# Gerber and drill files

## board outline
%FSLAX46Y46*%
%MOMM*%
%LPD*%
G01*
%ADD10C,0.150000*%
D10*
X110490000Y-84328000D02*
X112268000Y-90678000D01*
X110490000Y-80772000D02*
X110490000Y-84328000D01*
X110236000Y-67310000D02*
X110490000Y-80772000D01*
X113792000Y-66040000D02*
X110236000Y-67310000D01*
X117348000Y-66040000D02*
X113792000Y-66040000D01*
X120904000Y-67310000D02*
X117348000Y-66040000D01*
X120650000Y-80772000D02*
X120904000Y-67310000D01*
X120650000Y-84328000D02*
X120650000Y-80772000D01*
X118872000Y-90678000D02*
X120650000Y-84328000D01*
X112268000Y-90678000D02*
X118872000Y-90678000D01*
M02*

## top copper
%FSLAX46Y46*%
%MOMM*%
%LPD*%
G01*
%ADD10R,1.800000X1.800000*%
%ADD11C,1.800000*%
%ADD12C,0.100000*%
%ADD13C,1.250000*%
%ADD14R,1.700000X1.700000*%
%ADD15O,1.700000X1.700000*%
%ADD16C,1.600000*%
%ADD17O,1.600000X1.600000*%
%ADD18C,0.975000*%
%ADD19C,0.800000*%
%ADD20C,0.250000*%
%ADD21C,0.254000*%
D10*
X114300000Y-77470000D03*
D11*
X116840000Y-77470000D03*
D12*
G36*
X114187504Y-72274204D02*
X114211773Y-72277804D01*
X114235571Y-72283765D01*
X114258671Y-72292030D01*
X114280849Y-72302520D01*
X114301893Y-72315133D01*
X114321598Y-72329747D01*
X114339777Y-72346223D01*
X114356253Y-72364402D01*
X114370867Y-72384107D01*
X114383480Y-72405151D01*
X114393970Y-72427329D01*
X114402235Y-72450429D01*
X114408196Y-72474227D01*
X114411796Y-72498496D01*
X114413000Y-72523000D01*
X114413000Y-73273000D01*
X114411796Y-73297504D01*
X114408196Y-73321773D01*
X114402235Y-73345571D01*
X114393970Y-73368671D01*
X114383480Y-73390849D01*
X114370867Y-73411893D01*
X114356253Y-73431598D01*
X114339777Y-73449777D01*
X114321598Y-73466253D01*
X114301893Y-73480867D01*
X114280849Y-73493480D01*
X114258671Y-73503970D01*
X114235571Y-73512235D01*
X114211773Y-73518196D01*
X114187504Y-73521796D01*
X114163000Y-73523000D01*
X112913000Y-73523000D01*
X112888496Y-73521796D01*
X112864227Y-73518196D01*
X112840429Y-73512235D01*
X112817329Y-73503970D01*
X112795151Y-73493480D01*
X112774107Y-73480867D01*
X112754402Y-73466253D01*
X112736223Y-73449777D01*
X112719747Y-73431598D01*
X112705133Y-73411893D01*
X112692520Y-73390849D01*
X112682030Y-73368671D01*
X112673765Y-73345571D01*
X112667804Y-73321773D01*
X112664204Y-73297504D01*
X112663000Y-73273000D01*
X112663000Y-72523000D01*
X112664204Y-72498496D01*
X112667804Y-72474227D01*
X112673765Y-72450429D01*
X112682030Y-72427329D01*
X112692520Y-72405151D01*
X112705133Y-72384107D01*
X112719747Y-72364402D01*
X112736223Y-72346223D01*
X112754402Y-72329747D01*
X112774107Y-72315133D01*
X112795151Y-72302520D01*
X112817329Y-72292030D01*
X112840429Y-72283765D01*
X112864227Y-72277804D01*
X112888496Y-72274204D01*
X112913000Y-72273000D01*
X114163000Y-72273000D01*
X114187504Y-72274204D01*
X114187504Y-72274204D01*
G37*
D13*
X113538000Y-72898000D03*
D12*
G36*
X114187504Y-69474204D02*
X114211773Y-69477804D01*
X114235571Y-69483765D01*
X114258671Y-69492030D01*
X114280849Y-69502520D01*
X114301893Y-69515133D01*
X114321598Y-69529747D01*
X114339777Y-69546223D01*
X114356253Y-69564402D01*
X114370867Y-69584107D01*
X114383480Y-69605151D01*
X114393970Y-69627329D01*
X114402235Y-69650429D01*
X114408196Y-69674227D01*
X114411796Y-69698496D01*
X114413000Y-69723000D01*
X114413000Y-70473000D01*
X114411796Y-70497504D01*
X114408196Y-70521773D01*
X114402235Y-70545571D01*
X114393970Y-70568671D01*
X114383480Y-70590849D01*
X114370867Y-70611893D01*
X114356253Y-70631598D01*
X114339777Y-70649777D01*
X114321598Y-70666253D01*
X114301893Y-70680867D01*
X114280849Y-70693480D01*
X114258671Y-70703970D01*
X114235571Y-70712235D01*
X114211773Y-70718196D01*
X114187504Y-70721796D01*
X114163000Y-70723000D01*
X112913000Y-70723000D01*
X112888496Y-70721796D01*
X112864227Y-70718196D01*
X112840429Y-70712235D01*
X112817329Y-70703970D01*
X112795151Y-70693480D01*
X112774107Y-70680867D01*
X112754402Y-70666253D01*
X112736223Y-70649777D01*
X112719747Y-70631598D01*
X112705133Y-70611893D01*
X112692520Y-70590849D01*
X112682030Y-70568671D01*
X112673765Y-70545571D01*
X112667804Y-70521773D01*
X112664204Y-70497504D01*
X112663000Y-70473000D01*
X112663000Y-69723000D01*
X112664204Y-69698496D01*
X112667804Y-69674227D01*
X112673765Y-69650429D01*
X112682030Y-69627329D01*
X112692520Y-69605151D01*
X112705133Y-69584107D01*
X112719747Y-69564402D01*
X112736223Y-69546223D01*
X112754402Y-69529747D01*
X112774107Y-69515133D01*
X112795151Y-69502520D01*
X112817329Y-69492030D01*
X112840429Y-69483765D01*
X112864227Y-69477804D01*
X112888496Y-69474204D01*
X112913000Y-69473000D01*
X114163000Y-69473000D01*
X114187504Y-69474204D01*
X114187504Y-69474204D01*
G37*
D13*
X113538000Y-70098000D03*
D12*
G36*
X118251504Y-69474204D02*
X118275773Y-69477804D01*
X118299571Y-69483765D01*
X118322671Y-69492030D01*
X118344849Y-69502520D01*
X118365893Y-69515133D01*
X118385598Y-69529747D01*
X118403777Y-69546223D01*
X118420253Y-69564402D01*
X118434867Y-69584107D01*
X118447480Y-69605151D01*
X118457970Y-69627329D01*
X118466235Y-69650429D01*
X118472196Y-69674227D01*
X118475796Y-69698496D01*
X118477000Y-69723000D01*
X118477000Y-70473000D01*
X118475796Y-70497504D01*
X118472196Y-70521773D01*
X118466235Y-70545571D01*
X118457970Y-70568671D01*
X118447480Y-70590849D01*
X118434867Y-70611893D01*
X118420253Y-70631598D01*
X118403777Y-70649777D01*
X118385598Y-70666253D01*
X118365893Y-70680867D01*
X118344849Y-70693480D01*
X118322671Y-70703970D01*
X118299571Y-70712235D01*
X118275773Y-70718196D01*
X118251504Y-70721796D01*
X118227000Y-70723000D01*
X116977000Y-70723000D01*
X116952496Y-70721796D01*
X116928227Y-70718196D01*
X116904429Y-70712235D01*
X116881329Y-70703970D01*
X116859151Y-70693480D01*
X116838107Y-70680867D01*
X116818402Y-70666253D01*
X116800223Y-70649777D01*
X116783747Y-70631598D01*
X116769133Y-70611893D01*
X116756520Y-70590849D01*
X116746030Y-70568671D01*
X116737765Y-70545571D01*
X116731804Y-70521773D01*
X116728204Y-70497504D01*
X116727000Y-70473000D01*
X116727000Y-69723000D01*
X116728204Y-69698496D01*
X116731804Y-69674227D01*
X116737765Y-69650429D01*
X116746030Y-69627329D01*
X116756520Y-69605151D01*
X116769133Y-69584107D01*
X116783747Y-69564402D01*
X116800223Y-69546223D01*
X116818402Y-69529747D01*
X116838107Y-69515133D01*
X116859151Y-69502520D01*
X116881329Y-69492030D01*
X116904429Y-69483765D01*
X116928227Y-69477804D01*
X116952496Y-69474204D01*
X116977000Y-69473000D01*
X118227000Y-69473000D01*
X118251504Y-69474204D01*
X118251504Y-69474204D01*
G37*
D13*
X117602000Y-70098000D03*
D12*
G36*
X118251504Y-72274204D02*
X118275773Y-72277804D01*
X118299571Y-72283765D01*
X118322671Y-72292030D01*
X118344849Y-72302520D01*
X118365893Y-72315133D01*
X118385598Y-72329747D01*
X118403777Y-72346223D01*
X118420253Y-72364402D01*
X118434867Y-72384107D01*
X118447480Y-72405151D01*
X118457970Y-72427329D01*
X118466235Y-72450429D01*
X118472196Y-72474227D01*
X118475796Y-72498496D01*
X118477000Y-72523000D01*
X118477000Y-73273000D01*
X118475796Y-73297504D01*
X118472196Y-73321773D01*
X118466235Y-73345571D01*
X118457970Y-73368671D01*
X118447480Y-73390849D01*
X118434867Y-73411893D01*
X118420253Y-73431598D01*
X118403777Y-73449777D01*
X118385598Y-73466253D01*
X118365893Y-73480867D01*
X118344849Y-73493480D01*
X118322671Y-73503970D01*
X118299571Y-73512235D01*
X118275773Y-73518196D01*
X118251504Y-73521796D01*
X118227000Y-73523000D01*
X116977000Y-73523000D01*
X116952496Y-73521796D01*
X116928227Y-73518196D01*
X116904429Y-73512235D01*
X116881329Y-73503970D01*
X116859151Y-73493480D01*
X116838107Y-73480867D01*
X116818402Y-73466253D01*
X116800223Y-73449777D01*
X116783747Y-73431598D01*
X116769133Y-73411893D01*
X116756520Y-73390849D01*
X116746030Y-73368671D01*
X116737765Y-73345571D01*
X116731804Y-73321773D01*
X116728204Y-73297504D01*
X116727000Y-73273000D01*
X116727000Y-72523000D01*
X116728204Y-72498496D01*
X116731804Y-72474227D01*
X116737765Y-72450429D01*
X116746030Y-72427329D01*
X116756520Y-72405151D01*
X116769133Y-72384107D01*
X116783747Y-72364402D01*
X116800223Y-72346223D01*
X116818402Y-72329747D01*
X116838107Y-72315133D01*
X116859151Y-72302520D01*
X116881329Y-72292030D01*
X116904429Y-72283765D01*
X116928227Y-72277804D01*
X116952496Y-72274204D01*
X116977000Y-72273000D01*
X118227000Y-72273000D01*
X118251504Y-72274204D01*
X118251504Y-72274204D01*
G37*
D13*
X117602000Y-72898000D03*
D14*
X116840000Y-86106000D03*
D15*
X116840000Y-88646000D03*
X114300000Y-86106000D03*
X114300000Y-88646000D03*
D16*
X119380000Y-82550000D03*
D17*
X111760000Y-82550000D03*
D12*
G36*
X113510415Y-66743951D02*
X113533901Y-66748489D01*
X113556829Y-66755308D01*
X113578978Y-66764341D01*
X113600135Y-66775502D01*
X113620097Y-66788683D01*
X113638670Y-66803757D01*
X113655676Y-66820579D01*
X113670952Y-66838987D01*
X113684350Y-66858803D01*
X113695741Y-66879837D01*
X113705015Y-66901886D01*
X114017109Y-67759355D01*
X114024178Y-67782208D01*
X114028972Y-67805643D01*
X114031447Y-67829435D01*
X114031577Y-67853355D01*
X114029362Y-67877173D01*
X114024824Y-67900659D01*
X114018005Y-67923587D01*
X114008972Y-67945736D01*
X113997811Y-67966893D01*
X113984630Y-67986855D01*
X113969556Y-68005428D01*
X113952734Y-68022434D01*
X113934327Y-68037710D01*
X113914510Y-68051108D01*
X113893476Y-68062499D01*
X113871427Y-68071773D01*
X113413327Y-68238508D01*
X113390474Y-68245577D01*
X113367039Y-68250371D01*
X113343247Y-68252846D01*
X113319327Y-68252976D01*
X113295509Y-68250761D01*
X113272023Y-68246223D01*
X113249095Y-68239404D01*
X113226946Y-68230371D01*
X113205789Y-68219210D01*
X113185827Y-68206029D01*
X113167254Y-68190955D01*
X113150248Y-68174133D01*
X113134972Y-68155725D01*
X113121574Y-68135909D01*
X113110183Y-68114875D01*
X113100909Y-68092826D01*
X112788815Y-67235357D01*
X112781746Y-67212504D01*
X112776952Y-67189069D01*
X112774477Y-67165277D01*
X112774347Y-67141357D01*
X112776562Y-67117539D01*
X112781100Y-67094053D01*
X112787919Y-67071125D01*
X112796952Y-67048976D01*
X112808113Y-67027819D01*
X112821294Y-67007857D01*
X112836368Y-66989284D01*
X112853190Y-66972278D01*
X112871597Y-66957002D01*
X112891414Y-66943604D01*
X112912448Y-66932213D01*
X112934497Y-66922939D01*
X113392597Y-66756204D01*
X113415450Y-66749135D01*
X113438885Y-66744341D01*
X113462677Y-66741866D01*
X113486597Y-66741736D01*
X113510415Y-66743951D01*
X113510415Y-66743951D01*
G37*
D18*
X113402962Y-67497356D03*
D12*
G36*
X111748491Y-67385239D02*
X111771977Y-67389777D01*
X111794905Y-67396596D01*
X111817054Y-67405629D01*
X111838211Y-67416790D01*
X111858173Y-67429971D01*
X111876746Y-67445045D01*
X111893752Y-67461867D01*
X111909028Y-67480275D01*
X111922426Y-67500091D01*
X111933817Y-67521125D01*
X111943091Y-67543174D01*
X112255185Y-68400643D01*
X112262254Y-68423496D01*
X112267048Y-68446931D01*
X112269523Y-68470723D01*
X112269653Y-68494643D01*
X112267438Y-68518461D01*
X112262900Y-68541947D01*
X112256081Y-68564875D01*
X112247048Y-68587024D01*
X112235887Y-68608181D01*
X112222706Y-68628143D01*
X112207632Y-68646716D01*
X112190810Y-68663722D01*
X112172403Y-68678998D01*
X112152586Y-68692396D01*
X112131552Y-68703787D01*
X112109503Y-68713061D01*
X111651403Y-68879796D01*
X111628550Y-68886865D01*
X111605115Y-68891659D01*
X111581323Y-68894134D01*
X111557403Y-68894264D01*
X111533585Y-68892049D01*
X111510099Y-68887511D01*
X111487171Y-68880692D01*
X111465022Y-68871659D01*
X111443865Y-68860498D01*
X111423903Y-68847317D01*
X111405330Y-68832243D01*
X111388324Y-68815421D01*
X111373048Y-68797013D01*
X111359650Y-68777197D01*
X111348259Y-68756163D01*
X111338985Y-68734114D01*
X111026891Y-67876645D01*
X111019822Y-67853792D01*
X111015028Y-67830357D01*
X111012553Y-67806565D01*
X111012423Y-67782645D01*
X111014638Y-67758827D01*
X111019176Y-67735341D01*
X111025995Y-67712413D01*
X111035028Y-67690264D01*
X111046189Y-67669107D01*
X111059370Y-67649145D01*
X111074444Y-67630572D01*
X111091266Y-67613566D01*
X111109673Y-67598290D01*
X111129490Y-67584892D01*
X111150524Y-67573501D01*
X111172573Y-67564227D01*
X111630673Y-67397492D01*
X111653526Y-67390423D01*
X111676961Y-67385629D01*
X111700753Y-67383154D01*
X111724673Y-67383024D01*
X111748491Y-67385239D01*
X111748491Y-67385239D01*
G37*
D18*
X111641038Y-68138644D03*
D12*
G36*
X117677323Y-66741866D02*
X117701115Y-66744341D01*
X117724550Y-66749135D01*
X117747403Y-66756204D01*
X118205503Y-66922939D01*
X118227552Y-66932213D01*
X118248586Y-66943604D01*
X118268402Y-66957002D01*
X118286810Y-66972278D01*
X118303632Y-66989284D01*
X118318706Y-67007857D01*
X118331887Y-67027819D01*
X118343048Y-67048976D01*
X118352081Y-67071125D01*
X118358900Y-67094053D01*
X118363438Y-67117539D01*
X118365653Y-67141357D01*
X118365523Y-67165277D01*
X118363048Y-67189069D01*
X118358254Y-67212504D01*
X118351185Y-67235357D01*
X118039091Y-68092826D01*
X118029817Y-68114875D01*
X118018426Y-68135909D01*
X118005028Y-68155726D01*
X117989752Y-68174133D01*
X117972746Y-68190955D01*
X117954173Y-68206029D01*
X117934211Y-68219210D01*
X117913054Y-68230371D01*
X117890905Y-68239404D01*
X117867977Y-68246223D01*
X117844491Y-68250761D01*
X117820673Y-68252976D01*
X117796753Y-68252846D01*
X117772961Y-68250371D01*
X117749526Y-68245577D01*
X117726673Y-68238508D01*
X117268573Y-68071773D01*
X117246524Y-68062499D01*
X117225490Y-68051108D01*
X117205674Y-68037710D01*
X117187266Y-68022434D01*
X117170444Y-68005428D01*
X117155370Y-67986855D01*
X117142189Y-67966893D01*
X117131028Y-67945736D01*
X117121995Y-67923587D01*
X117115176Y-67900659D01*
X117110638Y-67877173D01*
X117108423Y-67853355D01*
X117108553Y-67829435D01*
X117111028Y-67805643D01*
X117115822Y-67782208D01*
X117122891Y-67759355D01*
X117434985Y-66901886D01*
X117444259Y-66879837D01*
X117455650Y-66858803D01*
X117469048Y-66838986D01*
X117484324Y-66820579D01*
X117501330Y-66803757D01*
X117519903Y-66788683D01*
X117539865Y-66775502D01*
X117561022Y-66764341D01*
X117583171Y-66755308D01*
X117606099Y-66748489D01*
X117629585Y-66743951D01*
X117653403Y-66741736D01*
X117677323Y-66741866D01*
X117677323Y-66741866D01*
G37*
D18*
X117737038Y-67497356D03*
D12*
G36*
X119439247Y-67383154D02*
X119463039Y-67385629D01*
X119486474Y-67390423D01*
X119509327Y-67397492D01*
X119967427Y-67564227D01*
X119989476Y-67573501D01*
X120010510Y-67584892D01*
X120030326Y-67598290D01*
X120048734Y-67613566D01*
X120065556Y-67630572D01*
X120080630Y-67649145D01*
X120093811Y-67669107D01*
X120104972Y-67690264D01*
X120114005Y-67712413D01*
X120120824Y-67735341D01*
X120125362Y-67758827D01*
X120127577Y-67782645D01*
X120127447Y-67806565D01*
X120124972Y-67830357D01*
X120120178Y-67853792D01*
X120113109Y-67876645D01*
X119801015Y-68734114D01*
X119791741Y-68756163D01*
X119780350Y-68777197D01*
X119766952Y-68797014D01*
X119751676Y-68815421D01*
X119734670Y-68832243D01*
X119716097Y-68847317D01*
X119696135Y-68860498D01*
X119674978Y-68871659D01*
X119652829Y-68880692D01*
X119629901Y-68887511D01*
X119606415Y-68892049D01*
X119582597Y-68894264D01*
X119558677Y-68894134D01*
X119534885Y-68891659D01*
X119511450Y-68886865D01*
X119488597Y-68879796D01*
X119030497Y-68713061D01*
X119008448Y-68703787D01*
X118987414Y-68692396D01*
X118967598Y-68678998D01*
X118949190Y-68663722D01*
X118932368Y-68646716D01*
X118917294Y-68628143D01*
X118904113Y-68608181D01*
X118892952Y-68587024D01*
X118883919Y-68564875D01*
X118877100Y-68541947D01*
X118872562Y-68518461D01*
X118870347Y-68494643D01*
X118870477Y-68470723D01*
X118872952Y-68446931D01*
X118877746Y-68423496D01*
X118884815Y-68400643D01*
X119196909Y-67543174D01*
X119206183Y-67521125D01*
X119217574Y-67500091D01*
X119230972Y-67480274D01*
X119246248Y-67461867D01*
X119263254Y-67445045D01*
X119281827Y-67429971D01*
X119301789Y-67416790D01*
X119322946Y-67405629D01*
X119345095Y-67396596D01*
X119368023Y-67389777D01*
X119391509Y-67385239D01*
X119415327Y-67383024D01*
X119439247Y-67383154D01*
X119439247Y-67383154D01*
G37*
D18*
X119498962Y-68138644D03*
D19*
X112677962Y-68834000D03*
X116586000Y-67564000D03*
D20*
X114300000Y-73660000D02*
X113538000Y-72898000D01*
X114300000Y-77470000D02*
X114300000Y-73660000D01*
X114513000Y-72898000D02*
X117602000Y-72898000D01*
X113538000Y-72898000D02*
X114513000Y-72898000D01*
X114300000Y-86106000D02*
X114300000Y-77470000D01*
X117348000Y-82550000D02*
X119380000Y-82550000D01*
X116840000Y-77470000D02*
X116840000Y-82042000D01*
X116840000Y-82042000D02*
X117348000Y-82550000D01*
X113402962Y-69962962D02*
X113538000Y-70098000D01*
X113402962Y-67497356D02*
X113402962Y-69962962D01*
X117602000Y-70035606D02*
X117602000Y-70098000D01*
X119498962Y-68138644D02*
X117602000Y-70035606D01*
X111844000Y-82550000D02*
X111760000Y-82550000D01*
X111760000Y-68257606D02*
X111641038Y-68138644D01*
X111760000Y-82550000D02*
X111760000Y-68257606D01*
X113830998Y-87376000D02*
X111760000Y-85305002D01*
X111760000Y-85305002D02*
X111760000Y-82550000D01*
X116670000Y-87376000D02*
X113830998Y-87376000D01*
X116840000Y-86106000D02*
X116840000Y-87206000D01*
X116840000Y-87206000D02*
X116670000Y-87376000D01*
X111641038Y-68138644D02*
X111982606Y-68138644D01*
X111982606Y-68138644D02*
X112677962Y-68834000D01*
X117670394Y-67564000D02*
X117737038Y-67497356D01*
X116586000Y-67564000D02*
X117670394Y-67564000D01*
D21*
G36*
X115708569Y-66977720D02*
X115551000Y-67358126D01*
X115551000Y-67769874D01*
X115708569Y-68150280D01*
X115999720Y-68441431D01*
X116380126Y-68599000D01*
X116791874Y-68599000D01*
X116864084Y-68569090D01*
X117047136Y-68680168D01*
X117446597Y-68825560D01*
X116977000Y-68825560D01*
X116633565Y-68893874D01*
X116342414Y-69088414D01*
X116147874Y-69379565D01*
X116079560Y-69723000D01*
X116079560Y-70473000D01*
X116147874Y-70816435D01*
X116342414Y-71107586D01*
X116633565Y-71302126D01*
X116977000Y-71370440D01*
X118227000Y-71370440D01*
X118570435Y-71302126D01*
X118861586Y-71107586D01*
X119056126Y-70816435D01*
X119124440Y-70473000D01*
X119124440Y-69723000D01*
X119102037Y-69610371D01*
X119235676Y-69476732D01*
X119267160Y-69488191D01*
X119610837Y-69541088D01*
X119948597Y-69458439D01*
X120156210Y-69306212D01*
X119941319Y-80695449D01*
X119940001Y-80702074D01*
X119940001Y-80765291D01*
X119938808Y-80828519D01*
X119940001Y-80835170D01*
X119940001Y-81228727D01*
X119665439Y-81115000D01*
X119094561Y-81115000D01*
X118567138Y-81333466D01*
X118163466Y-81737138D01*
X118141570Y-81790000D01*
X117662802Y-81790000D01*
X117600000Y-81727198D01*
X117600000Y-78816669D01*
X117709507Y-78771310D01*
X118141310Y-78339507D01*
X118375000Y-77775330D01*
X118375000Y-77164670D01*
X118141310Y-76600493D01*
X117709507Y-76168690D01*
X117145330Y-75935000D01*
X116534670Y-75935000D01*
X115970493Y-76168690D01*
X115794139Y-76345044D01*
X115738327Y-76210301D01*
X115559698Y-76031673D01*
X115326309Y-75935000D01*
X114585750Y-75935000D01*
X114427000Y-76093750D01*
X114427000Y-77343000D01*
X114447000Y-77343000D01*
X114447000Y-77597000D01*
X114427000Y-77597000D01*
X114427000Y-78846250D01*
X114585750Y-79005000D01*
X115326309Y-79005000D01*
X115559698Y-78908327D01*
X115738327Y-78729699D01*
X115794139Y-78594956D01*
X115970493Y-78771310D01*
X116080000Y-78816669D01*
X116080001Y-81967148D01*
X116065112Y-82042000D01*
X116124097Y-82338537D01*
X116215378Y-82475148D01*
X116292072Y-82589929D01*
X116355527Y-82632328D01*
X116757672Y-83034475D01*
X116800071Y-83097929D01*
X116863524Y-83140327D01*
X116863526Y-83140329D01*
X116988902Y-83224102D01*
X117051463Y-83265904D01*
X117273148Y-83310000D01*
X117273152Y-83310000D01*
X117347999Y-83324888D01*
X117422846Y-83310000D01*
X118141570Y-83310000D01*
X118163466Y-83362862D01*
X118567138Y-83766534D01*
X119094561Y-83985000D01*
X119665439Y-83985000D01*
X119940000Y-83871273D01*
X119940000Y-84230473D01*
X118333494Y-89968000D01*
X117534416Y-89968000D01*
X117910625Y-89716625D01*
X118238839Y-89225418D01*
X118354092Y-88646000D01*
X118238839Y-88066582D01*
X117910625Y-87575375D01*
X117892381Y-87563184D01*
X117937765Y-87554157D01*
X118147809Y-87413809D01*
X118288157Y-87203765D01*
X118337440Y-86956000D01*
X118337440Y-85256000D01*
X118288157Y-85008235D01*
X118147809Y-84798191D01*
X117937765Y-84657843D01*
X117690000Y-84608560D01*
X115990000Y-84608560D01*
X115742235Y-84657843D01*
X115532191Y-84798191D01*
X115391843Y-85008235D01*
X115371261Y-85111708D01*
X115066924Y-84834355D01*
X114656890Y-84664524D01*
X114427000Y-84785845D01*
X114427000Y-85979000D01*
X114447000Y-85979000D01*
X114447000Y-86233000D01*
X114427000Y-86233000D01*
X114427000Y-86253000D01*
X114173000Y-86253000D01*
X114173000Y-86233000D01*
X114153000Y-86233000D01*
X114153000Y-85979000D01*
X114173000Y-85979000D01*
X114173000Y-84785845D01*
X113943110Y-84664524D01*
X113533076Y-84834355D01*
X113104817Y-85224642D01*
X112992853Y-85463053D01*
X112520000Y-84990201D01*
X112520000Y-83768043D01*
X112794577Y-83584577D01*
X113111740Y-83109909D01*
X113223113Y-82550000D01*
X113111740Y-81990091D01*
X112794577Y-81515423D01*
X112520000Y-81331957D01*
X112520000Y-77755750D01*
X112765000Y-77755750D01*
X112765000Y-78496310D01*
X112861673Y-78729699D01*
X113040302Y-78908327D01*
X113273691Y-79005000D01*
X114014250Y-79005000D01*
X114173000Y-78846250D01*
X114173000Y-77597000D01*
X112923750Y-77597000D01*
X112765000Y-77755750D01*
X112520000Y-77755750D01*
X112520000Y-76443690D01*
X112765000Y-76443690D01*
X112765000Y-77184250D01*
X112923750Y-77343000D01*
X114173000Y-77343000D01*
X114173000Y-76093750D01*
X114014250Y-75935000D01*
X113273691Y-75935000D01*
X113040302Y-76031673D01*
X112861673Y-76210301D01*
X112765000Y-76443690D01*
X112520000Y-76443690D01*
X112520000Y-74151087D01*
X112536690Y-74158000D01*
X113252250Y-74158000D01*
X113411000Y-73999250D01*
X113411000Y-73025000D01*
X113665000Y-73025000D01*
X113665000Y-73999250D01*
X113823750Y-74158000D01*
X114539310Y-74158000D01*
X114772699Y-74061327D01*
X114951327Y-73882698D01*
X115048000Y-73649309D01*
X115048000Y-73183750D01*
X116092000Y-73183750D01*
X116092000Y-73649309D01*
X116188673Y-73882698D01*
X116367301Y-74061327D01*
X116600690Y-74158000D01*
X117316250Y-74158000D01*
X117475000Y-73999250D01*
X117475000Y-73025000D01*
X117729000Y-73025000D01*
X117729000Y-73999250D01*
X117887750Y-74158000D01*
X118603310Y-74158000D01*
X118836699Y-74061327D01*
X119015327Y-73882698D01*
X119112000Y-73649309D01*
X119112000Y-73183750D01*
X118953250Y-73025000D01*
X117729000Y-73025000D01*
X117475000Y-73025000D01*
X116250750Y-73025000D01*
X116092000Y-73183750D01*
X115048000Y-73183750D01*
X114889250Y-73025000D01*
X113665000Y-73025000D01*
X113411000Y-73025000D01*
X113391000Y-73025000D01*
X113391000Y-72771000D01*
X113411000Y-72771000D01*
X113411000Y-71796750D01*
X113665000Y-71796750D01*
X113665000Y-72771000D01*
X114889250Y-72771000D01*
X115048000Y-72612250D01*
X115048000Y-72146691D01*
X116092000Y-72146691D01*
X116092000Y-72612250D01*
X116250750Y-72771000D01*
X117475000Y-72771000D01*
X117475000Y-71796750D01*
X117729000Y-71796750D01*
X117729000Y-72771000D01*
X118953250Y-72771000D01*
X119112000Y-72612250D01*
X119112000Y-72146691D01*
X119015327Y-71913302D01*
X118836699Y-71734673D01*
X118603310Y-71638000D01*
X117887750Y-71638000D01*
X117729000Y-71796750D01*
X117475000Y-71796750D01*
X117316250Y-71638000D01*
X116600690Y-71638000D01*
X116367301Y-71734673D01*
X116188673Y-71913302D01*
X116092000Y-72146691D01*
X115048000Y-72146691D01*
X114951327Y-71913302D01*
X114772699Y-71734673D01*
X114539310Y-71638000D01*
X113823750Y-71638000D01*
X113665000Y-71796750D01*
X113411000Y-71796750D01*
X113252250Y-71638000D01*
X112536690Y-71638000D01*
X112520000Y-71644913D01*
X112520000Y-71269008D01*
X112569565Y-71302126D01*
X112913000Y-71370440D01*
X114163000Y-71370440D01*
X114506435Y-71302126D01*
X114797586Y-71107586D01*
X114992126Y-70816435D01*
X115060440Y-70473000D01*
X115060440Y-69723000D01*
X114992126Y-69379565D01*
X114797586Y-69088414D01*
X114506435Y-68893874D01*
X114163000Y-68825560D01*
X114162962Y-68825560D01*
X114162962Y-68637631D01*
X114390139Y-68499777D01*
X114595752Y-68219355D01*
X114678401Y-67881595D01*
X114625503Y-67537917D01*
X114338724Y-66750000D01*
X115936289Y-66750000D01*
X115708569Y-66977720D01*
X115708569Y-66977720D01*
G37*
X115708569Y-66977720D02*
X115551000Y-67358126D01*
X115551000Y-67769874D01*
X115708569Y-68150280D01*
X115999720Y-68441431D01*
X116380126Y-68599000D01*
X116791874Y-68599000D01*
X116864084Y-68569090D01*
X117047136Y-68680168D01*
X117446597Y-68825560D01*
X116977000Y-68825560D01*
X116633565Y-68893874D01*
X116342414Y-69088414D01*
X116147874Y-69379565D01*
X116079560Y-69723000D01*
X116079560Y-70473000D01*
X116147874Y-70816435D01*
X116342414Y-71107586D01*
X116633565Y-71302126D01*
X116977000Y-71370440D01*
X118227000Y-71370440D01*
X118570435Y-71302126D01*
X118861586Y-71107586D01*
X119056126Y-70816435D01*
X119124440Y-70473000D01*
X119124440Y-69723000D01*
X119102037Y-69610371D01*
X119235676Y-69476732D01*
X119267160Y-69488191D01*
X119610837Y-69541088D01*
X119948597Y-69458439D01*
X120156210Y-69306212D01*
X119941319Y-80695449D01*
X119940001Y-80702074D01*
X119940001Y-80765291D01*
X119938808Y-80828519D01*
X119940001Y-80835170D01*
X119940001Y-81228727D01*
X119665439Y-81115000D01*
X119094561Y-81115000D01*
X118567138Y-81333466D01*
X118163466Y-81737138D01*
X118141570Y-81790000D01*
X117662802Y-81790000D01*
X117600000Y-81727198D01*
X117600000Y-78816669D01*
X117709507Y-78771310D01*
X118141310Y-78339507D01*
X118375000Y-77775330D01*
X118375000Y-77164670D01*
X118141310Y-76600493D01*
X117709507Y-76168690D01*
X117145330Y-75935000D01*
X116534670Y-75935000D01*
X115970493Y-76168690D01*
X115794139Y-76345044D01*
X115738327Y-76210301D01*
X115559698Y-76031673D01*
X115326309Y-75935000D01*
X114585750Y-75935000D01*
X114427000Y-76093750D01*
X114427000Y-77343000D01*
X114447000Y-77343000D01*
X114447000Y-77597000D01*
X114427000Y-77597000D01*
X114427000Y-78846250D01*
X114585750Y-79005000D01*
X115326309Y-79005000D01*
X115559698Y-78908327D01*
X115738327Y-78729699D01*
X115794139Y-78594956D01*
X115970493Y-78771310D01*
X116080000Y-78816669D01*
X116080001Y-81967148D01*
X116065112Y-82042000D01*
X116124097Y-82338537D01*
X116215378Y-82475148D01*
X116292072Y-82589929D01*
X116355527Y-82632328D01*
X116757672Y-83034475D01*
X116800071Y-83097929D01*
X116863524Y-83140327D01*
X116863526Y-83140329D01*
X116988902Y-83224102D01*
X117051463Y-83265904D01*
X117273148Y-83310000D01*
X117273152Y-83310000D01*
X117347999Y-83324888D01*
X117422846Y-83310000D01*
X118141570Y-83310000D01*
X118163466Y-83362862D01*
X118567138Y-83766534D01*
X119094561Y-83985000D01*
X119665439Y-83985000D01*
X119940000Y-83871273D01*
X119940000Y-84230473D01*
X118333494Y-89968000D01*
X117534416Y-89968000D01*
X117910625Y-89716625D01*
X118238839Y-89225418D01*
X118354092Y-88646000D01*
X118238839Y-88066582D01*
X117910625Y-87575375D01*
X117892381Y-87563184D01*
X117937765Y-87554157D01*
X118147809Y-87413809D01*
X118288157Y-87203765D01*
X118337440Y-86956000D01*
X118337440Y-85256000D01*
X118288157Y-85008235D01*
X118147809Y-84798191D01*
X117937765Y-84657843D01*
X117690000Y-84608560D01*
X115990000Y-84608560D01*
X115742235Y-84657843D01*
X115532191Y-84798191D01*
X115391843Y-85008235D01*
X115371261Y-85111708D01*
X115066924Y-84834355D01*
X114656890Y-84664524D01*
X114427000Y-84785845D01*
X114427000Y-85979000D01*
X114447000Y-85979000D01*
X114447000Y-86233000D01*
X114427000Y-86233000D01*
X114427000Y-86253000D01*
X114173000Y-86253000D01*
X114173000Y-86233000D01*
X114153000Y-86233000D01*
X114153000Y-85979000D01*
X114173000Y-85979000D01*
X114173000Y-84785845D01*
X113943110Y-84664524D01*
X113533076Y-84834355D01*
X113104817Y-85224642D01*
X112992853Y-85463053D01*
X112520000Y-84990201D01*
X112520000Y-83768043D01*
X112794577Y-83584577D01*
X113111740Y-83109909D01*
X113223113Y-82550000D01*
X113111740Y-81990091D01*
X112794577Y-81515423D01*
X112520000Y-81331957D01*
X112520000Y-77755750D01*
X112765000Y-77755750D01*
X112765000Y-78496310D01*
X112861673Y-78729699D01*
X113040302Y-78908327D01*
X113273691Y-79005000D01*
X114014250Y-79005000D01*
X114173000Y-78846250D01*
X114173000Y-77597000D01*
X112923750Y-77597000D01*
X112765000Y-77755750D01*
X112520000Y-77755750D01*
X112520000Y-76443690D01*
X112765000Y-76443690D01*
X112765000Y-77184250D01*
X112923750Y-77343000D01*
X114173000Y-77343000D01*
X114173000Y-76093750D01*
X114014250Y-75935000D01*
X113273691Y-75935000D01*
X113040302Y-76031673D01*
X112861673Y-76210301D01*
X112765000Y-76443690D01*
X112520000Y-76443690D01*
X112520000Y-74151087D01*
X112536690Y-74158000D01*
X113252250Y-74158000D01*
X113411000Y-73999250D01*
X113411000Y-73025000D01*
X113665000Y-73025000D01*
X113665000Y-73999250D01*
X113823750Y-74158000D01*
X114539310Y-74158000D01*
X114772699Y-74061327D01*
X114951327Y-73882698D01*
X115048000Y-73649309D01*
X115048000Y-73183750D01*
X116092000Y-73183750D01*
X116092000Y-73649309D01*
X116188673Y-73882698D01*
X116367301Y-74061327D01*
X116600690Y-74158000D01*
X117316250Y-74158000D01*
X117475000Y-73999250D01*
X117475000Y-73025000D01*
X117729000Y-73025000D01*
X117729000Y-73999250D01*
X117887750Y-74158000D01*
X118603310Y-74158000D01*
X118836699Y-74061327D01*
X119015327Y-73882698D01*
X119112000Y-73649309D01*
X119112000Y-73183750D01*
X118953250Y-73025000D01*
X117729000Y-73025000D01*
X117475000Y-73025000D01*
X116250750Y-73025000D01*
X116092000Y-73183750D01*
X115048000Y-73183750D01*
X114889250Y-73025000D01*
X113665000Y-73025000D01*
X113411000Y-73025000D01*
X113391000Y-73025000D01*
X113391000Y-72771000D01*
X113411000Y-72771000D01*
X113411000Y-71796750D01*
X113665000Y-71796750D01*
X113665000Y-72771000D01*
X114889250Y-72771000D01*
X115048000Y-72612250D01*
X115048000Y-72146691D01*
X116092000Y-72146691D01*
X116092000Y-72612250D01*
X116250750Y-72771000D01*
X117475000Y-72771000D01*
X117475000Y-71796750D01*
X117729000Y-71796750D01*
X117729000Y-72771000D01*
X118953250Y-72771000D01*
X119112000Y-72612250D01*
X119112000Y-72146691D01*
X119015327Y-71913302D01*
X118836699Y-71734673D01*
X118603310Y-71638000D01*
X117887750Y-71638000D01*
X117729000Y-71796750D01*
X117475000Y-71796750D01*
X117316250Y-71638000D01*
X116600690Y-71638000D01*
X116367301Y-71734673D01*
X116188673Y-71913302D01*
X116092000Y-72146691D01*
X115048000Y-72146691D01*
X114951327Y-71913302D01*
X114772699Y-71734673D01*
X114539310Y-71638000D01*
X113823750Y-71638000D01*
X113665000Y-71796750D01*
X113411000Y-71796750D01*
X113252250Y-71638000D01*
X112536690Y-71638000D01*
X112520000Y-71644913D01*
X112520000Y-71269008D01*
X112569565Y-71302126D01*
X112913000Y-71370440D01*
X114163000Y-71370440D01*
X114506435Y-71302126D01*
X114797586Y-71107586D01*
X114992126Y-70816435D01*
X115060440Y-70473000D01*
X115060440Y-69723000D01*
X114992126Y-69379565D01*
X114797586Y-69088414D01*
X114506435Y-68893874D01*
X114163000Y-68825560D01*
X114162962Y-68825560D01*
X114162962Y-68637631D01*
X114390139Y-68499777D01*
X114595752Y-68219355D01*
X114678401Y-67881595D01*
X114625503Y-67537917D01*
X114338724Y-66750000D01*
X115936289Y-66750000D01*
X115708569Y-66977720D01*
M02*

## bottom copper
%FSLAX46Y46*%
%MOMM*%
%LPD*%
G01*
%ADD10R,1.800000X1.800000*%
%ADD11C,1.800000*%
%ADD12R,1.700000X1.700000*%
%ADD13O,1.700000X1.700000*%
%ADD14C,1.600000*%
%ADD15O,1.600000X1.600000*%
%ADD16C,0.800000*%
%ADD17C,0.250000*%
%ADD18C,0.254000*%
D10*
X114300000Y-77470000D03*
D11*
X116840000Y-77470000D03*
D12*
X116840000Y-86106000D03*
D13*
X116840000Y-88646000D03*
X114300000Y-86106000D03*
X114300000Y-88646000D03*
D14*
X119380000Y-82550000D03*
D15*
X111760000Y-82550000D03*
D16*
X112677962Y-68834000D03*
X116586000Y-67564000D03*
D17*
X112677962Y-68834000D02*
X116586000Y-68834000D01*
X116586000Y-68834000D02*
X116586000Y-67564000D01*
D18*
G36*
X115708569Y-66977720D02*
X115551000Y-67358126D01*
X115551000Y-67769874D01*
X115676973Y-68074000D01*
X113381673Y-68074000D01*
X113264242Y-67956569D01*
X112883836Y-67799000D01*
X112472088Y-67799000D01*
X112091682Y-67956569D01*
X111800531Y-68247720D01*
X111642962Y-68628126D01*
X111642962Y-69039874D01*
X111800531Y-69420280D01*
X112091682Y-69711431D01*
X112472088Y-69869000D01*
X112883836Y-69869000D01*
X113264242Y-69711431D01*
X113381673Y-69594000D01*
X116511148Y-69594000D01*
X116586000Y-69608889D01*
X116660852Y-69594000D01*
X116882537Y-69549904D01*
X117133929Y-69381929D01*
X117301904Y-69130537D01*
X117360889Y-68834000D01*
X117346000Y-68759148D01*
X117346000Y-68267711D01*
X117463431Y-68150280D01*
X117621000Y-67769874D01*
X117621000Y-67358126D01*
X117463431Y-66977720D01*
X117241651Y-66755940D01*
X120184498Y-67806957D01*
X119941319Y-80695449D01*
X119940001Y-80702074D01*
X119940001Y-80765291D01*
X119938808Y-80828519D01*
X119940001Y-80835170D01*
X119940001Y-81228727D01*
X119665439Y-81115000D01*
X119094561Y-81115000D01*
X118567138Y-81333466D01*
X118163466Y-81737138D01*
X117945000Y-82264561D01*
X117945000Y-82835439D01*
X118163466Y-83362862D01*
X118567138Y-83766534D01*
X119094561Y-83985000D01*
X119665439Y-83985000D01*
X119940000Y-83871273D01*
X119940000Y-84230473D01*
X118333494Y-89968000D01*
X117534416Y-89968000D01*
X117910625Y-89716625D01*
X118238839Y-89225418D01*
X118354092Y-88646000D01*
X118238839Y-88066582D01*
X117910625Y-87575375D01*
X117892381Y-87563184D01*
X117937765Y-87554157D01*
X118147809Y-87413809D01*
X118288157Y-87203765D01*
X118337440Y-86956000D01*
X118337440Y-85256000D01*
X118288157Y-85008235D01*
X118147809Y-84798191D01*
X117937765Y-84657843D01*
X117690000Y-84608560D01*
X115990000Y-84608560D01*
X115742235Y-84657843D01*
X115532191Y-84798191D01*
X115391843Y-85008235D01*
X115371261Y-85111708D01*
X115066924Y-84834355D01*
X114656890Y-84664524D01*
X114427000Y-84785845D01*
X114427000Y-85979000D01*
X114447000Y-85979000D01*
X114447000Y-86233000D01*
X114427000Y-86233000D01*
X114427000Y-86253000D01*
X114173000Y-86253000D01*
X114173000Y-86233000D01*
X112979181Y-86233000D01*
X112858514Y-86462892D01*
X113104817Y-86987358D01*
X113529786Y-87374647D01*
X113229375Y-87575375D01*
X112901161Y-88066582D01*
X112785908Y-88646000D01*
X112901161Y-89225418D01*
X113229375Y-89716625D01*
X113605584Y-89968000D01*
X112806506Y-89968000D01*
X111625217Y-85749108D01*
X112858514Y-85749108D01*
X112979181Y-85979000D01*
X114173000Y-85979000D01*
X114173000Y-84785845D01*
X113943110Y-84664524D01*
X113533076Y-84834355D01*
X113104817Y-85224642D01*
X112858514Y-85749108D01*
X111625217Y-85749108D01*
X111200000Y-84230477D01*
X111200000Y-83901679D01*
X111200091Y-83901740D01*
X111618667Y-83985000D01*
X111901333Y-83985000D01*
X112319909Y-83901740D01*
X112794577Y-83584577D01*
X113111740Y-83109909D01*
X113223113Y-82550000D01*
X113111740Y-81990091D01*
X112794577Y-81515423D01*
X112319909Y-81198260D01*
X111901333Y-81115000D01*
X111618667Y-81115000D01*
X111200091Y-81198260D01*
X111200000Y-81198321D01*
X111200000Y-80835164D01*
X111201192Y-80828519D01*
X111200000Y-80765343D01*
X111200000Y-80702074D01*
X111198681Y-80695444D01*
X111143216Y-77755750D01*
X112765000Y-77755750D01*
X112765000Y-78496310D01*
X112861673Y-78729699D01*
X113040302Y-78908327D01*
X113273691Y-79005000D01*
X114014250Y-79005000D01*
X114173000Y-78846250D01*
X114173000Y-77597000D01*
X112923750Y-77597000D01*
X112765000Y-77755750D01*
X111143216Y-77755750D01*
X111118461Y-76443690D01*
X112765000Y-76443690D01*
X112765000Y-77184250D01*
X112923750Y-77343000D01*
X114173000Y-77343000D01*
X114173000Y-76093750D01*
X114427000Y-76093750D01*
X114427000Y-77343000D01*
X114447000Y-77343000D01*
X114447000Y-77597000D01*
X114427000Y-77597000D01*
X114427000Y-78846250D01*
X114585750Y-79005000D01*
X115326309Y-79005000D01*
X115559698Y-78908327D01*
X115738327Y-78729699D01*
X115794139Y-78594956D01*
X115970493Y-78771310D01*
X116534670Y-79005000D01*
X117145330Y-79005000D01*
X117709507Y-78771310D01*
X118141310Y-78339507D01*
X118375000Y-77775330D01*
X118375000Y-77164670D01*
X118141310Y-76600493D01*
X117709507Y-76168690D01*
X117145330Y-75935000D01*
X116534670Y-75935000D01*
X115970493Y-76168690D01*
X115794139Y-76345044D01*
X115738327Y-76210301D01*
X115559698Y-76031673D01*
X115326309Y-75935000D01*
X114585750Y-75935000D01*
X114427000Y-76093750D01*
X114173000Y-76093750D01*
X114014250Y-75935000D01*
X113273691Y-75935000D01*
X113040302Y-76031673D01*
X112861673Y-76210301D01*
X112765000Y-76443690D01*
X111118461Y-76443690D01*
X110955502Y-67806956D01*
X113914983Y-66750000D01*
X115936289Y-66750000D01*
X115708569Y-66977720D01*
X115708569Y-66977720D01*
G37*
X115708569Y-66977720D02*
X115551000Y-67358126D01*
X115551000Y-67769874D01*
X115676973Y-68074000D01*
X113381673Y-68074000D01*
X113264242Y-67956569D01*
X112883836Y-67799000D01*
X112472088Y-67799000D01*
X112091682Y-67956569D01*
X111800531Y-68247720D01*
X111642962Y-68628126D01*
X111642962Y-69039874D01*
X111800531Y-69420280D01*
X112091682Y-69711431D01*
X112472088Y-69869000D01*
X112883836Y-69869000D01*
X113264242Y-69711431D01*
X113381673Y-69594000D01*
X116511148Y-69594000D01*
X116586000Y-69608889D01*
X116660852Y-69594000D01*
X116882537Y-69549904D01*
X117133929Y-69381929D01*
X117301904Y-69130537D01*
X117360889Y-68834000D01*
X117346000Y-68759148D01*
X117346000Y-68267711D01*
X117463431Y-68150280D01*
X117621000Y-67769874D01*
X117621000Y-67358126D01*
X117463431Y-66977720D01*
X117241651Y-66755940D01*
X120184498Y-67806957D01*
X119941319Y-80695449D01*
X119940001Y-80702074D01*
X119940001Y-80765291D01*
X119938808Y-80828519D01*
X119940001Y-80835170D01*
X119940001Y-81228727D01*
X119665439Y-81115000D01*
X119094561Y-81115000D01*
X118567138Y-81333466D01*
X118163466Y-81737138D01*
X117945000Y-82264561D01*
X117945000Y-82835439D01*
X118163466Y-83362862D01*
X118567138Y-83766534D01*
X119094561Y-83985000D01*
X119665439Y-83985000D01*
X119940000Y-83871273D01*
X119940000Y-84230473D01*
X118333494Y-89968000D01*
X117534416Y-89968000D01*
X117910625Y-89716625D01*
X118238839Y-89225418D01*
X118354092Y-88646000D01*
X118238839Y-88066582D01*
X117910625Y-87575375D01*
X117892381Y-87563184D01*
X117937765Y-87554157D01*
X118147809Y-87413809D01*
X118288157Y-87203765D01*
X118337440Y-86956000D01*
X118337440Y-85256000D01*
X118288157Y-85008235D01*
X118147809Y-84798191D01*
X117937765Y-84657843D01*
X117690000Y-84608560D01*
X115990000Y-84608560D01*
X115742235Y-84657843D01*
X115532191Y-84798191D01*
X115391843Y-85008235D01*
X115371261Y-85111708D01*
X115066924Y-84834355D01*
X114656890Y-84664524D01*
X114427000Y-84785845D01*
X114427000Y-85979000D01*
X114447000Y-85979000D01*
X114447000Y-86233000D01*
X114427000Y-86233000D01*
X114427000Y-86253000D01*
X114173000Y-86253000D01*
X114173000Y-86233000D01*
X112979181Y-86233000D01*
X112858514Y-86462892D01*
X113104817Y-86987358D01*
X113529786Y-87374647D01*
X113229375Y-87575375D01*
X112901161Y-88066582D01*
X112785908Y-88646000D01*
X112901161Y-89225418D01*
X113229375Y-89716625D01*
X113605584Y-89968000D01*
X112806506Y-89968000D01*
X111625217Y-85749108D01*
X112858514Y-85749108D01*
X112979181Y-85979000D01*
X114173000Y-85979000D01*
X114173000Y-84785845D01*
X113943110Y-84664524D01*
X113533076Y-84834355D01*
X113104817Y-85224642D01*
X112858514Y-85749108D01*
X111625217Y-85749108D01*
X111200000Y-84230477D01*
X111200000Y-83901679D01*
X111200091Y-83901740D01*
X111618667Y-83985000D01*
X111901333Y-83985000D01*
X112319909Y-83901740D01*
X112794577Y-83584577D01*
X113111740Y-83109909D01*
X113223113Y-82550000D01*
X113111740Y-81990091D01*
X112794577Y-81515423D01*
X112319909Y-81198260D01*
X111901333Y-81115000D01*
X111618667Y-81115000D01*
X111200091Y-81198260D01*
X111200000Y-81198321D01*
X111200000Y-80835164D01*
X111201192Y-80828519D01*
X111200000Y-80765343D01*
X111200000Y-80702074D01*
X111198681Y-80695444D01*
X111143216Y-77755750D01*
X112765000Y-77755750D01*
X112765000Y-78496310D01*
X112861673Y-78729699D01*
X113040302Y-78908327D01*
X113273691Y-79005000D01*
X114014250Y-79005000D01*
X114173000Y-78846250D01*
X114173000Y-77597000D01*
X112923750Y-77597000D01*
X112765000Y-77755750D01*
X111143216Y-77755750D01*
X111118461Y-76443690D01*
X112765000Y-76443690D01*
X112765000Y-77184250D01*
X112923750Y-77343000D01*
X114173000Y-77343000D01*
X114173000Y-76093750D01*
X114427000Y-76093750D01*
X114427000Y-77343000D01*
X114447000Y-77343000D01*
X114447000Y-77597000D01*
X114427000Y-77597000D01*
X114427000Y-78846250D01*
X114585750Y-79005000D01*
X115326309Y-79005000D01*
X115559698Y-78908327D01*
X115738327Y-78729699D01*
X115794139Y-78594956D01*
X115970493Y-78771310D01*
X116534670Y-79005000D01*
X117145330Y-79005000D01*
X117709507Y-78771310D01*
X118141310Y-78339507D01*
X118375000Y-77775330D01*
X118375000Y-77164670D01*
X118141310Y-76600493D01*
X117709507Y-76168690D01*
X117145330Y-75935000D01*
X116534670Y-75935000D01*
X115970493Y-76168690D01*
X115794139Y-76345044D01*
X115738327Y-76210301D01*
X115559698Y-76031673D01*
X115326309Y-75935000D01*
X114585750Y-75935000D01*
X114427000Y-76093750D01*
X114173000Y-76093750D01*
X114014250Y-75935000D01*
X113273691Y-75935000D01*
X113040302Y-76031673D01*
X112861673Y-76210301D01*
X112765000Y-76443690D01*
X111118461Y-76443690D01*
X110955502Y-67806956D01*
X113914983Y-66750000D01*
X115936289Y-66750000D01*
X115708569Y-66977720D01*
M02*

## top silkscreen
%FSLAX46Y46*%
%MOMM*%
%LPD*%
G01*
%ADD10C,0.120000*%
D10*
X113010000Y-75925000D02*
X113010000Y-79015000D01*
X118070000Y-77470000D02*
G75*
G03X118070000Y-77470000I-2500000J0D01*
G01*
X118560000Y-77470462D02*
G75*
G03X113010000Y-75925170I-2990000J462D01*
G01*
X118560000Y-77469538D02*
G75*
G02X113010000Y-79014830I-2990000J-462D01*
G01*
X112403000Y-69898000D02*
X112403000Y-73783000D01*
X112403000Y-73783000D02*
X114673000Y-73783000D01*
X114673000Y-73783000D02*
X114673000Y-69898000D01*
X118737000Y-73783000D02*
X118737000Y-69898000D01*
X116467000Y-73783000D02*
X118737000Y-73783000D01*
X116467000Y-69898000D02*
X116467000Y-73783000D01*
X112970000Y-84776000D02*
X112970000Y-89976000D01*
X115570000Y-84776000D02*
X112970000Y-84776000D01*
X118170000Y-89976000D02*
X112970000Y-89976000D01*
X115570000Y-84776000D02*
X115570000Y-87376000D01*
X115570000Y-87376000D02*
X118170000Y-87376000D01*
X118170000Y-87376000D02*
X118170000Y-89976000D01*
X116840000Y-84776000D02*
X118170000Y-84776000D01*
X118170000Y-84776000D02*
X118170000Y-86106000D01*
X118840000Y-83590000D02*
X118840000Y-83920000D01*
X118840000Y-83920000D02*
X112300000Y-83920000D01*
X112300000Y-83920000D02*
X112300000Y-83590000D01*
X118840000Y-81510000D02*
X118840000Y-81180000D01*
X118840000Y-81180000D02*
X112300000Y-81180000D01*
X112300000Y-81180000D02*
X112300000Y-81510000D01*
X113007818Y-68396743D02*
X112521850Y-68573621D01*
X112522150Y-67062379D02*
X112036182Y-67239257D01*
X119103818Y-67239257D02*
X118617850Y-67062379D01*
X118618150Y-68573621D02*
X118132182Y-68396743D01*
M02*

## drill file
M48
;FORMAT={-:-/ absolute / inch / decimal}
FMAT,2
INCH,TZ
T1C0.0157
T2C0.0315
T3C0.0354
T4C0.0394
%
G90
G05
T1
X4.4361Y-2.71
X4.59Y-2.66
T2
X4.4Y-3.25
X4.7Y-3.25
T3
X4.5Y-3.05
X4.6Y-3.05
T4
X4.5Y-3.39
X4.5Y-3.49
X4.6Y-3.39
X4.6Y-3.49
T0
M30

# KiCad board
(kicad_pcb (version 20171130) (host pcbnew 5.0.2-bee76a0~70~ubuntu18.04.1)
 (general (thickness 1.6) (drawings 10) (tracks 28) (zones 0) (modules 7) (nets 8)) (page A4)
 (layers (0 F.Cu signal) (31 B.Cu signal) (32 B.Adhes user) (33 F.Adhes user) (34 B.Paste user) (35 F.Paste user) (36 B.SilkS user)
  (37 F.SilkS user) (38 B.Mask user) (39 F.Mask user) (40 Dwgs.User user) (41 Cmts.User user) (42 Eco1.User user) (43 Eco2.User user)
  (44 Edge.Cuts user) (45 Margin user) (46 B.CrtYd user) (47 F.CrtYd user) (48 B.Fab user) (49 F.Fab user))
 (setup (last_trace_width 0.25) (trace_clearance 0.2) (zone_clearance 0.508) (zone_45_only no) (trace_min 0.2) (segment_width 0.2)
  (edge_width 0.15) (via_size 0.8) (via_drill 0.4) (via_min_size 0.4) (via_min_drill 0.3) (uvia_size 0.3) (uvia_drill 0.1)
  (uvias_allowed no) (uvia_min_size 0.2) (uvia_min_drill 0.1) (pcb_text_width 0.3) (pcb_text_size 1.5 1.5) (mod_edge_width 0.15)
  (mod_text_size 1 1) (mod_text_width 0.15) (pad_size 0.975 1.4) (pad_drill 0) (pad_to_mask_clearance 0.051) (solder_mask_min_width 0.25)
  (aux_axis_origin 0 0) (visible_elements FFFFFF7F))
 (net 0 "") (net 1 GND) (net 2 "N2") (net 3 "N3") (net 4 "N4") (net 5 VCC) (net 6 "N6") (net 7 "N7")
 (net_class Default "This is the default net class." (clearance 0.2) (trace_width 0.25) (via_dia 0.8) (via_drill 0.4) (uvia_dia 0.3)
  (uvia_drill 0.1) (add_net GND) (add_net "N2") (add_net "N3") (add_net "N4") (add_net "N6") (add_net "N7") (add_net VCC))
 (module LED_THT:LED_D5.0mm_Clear (layer F.Cu) (at 114.3 77.47)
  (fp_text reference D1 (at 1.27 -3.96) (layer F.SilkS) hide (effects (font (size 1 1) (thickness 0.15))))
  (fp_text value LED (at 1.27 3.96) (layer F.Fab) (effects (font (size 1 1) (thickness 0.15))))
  (fp_line (start -1.29 -1.545) (end -1.29 1.545) (layer F.SilkS) (width 0.12))
  (fp_circle (center 1.27 0) (end 3.77 0) (layer F.SilkS) (width 0.12))
  (fp_arc (start 1.27 0) (end -1.29 -1.54483) (angle 148.9) (layer F.SilkS) (width 0.12))
  (fp_arc (start 1.27 0) (end -1.29 1.54483) (angle -148.9) (layer F.SilkS) (width 0.12))
  (pad 1 thru_hole rect (at 0 0) (size 1.8 1.8) (drill 0.9) (layers *.Cu *.Mask) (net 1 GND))
  (pad 2 thru_hole circle (at 2.54 0) (size 1.8 1.8) (drill 0.9) (layers *.Cu *.Mask) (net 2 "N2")))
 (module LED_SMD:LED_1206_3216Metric (layer F.Cu) (at 113.538 71.498 90)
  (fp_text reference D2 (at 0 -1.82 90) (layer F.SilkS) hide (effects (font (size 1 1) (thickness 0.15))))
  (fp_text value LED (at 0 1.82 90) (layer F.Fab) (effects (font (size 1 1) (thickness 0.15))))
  (fp_line (start 1.6 -1.135) (end -2.285 -1.135) (layer F.SilkS) (width 0.12))
  (fp_line (start -2.285 -1.135) (end -2.285 1.135) (layer F.SilkS) (width 0.12))
  (fp_line (start -2.285 1.135) (end 1.6 1.135) (layer F.SilkS) (width 0.12))
  (pad 1 smd roundrect (at -1.4 0 90) (size 1.25 1.75) (layers F.Cu F.Paste F.Mask) (roundrect_rratio 0.2) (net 1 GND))
  (pad 2 smd roundrect (at 1.4 0 90) (size 1.25 1.75) (layers F.Cu F.Paste F.Mask) (roundrect_rratio 0.2) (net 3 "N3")))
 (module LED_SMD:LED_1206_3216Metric (layer F.Cu) (at 117.602 71.498 90)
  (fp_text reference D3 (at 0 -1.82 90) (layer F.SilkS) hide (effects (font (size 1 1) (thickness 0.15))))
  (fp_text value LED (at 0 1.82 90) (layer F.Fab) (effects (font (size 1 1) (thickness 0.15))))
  (fp_line (start -2.285 1.135) (end 1.6 1.135) (layer F.SilkS) (width 0.12))
  (fp_line (start -2.285 -1.135) (end -2.285 1.135) (layer F.SilkS) (width 0.12))
  (fp_line (start 1.6 -1.135) (end -2.285 -1.135) (layer F.SilkS) (width 0.12))
  (pad 2 smd roundrect (at 1.4 0 90) (size 1.25 1.75) (layers F.Cu F.Paste F.Mask) (roundrect_rratio 0.2) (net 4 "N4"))
  (pad 1 smd roundrect (at -1.4 0 90) (size 1.25 1.75) (layers F.Cu F.Paste F.Mask) (roundrect_rratio 0.2) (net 1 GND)))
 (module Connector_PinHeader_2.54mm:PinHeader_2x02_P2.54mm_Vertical (layer F.Cu) (at 116.84 86.106 270)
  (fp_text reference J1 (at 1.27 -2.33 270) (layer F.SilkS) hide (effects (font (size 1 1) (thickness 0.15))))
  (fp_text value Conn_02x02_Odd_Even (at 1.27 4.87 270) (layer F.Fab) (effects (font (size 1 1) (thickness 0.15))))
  (fp_line (start -1.33 3.87) (end 3.87 3.87) (layer F.SilkS) (width 0.12))
  (fp_line (start -1.33 1.27) (end -1.33 3.87) (layer F.SilkS) (width 0.12))
  (fp_line (start 3.87 -1.33) (end 3.87 3.87) (layer F.SilkS) (width 0.12))
  (fp_line (start -1.33 1.27) (end 1.27 1.27) (layer F.SilkS) (width 0.12))
  (fp_line (start 1.27 1.27) (end 1.27 -1.33) (layer F.SilkS) (width 0.12))
  (fp_line (start 1.27 -1.33) (end 3.87 -1.33) (layer F.SilkS) (width 0.12))
  (fp_line (start -1.33 0) (end -1.33 -1.33) (layer F.SilkS) (width 0.12))
  (fp_line (start -1.33 -1.33) (end 0 -1.33) (layer F.SilkS) (width 0.12))
  (pad 1 thru_hole rect (at 0 0 270) (size 1.7 1.7) (drill 1) (layers *.Cu *.Mask) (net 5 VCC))
  (pad 2 thru_hole oval (at 2.54 0 270) (size 1.7 1.7) (drill 1) (layers *.Cu *.Mask) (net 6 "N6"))
  (pad 3 thru_hole oval (at 0 2.54 270) (size 1.7 1.7) (drill 1) (layers *.Cu *.Mask) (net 1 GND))
  (pad 4 thru_hole oval (at 2.54 2.54 270) (size 1.7 1.7) (drill 1) (layers *.Cu *.Mask) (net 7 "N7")))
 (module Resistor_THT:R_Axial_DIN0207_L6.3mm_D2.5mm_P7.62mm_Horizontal (layer F.Cu) (at 119.38 82.55 180)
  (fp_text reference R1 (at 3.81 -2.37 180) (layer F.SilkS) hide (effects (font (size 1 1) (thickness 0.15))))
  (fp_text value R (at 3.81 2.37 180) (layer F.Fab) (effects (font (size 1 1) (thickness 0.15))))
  (fp_line (start 0.54 -1.04) (end 0.54 -1.37) (layer F.SilkS) (width 0.12))
  (fp_line (start 0.54 -1.37) (end 7.08 -1.37) (layer F.SilkS) (width 0.12))
  (fp_line (start 7.08 -1.37) (end 7.08 -1.04) (layer F.SilkS) (width 0.12))
  (fp_line (start 0.54 1.04) (end 0.54 1.37) (layer F.SilkS) (width 0.12))
  (fp_line (start 0.54 1.37) (end 7.08 1.37) (layer F.SilkS) (width 0.12))
  (fp_line (start 7.08 1.37) (end 7.08 1.04) (layer F.SilkS) (width 0.12))
  (pad 1 thru_hole circle (at 0 0 180) (size 1.6 1.6) (drill 0.8) (layers *.Cu *.Mask) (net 2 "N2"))
  (pad 2 thru_hole oval (at 7.62 0 180) (size 1.6 1.6) (drill 0.8) (layers *.Cu *.Mask) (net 5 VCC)))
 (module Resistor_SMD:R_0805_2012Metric (layer F.Cu) (at 112.522 67.818 200)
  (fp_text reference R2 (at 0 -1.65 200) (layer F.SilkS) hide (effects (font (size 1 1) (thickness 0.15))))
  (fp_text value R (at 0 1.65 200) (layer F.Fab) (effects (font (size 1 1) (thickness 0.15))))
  (fp_line (start -0.258578 -0.71) (end 0.258579 -0.71) (layer F.SilkS) (width 0.12))
  (fp_line (start -0.258579 0.71) (end 0.258578 0.71) (layer F.SilkS) (width 0.12))
  (pad 1 smd roundrect (at -0.9375 0 200) (size 0.975 1.4) (layers F.Cu F.Paste F.Mask) (roundrect_rratio 0.25) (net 3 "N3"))
  (pad 2 smd roundrect (at 0.9375 0 200) (size 0.975 1.4) (layers F.Cu F.Paste F.Mask) (roundrect_rratio 0.25) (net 5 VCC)))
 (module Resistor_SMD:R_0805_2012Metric (layer F.Cu) (at 118.618 67.818 160)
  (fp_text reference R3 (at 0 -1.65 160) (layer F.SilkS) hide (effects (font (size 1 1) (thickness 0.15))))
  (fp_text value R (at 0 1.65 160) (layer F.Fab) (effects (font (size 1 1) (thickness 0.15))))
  (fp_line (start -0.258578 0.71) (end 0.258578 0.71) (layer F.SilkS) (width 0.12))
  (fp_line (start -0.258578 -0.71) (end 0.258578 -0.71) (layer F.SilkS) (width 0.12))
  (pad 2 smd roundrect (at 0.9375 0 160) (size 0.975 1.4) (layers F.Cu F.Paste F.Mask) (roundrect_rratio 0.25) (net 5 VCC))
  (pad 1 smd roundrect (at -0.9375 0 160) (size 0.975 1.4) (layers F.Cu F.Paste F.Mask) (roundrect_rratio 0.25) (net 4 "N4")))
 (gr_line (start 110.49 84.328) (end 112.268 90.678) (layer Edge.Cuts) (width 0.15))
 (gr_line (start 110.49 80.772) (end 110.49 84.328) (layer Edge.Cuts) (width 0.15))
 (gr_line (start 110.236 67.31) (end 110.49 80.772) (layer Edge.Cuts) (width 0.15))
 (gr_line (start 113.792 66.04) (end 110.236 67.31) (layer Edge.Cuts) (width 0.15))
 (gr_line (start 117.348 66.04) (end 113.792 66.04) (layer Edge.Cuts) (width 0.15))
 (gr_line (start 120.904 67.31) (end 117.348 66.04) (layer Edge.Cuts) (width 0.15))
 (gr_line (start 120.65 80.772) (end 120.904 67.31) (layer Edge.Cuts) (width 0.15))
 (gr_line (start 120.65 84.328) (end 120.65 80.772) (layer Edge.Cuts) (width 0.15))
 (gr_line (start 118.872 90.678) (end 120.65 84.328) (layer Edge.Cuts) (width 0.15))
 (gr_line (start 112.268 90.678) (end 118.872 90.678) (layer Edge.Cuts) (width 0.15))
 (segment (start 114.3 73.66) (end 113.538 72.898) (width 0.25) (layer F.Cu) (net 1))
 (segment (start 114.3 77.47) (end 114.3 73.66) (width 0.25) (layer F.Cu) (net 1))
 (segment (start 114.513 72.898) (end 117.602 72.898) (width 0.25) (layer F.Cu) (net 1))
 (segment (start 113.538 72.898) (end 114.513 72.898) (width 0.25) (layer F.Cu) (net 1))
 (segment (start 114.3 86.106) (end 114.3 77.47) (width 0.25) (layer F.Cu) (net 1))
 (segment (start 117.348 82.55) (end 119.38 82.55) (width 0.25) (layer F.Cu) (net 2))
 (segment (start 116.84 77.47) (end 116.84 82.042) (width 0.25) (layer F.Cu) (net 2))
 (segment (start 116.84 82.042) (end 117.348 82.55) (width 0.25) (layer F.Cu) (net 2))
 (segment (start 113.402962 69.962962) (end 113.538 70.098) (width 0.25) (layer F.Cu) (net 3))
 (segment (start 113.402962 67.497356) (end 113.402962 69.962962) (width 0.25) (layer F.Cu) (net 3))
 (segment (start 117.602 70.035606) (end 117.602 70.098) (width 0.25) (layer F.Cu) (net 4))
 (segment (start 119.498962 68.138644) (end 117.602 70.035606) (width 0.25) (layer F.Cu) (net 4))
 (segment (start 111.844 82.55) (end 111.76 82.55) (width 0.25) (layer F.Cu) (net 5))
 (segment (start 111.76 68.257606) (end 111.641038 68.138644) (width 0.25) (layer F.Cu) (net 5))
 (segment (start 111.76 82.55) (end 111.76 68.257606) (width 0.25) (layer F.Cu) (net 5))
 (segment (start 113.830998 87.376) (end 111.76 85.305002) (width 0.25) (layer F.Cu) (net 5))
 (segment (start 111.76 85.305002) (end 111.76 82.55) (width 0.25) (layer F.Cu) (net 5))
 (segment (start 116.67 87.376) (end 113.830998 87.376) (width 0.25) (layer F.Cu) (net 5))
 (segment (start 116.84 86.106) (end 116.84 87.206) (width 0.25) (layer F.Cu) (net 5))
 (segment (start 116.84 87.206) (end 116.67 87.376) (width 0.25) (layer F.Cu) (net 5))
 (segment (start 111.641038 68.138644) (end 111.982606 68.138644) (width 0.25) (layer F.Cu) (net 5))
 (via (at 112.677962 68.834) (size 0.8) (drill 0.4) (layers F.Cu B.Cu) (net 5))
 (segment (start 111.982606 68.138644) (end 112.677962 68.834) (width 0.25) (layer F.Cu) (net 5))
 (segment (start 112.677962 68.834) (end 116.586 68.834) (width 0.25) (layer B.Cu) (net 5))
 (via (at 116.586 67.564) (size 0.8) (drill 0.4) (layers F.Cu B.Cu) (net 5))
 (segment (start 116.586 68.834) (end 116.586 67.564) (width 0.25) (layer B.Cu) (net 5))
 (segment (start 117.670394 67.564) (end 117.737038 67.497356) (width 0.25) (layer F.Cu) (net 5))
 (segment (start 116.586 67.564) (end 117.670394 67.564) (width 0.25) (layer F.Cu) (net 5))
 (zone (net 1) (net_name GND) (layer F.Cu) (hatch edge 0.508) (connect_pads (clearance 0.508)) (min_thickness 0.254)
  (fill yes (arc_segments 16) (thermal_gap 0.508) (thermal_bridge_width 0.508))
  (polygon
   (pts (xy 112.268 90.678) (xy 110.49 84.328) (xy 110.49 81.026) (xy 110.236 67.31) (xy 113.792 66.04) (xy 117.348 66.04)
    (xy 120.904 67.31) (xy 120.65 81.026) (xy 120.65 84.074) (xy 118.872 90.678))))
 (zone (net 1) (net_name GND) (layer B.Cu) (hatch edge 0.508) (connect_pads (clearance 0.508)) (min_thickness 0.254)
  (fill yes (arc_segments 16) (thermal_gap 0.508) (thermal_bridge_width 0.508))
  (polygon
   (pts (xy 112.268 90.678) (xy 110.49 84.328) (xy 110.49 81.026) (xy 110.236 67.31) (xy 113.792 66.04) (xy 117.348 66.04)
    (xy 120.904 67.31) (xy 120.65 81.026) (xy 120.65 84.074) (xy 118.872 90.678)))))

